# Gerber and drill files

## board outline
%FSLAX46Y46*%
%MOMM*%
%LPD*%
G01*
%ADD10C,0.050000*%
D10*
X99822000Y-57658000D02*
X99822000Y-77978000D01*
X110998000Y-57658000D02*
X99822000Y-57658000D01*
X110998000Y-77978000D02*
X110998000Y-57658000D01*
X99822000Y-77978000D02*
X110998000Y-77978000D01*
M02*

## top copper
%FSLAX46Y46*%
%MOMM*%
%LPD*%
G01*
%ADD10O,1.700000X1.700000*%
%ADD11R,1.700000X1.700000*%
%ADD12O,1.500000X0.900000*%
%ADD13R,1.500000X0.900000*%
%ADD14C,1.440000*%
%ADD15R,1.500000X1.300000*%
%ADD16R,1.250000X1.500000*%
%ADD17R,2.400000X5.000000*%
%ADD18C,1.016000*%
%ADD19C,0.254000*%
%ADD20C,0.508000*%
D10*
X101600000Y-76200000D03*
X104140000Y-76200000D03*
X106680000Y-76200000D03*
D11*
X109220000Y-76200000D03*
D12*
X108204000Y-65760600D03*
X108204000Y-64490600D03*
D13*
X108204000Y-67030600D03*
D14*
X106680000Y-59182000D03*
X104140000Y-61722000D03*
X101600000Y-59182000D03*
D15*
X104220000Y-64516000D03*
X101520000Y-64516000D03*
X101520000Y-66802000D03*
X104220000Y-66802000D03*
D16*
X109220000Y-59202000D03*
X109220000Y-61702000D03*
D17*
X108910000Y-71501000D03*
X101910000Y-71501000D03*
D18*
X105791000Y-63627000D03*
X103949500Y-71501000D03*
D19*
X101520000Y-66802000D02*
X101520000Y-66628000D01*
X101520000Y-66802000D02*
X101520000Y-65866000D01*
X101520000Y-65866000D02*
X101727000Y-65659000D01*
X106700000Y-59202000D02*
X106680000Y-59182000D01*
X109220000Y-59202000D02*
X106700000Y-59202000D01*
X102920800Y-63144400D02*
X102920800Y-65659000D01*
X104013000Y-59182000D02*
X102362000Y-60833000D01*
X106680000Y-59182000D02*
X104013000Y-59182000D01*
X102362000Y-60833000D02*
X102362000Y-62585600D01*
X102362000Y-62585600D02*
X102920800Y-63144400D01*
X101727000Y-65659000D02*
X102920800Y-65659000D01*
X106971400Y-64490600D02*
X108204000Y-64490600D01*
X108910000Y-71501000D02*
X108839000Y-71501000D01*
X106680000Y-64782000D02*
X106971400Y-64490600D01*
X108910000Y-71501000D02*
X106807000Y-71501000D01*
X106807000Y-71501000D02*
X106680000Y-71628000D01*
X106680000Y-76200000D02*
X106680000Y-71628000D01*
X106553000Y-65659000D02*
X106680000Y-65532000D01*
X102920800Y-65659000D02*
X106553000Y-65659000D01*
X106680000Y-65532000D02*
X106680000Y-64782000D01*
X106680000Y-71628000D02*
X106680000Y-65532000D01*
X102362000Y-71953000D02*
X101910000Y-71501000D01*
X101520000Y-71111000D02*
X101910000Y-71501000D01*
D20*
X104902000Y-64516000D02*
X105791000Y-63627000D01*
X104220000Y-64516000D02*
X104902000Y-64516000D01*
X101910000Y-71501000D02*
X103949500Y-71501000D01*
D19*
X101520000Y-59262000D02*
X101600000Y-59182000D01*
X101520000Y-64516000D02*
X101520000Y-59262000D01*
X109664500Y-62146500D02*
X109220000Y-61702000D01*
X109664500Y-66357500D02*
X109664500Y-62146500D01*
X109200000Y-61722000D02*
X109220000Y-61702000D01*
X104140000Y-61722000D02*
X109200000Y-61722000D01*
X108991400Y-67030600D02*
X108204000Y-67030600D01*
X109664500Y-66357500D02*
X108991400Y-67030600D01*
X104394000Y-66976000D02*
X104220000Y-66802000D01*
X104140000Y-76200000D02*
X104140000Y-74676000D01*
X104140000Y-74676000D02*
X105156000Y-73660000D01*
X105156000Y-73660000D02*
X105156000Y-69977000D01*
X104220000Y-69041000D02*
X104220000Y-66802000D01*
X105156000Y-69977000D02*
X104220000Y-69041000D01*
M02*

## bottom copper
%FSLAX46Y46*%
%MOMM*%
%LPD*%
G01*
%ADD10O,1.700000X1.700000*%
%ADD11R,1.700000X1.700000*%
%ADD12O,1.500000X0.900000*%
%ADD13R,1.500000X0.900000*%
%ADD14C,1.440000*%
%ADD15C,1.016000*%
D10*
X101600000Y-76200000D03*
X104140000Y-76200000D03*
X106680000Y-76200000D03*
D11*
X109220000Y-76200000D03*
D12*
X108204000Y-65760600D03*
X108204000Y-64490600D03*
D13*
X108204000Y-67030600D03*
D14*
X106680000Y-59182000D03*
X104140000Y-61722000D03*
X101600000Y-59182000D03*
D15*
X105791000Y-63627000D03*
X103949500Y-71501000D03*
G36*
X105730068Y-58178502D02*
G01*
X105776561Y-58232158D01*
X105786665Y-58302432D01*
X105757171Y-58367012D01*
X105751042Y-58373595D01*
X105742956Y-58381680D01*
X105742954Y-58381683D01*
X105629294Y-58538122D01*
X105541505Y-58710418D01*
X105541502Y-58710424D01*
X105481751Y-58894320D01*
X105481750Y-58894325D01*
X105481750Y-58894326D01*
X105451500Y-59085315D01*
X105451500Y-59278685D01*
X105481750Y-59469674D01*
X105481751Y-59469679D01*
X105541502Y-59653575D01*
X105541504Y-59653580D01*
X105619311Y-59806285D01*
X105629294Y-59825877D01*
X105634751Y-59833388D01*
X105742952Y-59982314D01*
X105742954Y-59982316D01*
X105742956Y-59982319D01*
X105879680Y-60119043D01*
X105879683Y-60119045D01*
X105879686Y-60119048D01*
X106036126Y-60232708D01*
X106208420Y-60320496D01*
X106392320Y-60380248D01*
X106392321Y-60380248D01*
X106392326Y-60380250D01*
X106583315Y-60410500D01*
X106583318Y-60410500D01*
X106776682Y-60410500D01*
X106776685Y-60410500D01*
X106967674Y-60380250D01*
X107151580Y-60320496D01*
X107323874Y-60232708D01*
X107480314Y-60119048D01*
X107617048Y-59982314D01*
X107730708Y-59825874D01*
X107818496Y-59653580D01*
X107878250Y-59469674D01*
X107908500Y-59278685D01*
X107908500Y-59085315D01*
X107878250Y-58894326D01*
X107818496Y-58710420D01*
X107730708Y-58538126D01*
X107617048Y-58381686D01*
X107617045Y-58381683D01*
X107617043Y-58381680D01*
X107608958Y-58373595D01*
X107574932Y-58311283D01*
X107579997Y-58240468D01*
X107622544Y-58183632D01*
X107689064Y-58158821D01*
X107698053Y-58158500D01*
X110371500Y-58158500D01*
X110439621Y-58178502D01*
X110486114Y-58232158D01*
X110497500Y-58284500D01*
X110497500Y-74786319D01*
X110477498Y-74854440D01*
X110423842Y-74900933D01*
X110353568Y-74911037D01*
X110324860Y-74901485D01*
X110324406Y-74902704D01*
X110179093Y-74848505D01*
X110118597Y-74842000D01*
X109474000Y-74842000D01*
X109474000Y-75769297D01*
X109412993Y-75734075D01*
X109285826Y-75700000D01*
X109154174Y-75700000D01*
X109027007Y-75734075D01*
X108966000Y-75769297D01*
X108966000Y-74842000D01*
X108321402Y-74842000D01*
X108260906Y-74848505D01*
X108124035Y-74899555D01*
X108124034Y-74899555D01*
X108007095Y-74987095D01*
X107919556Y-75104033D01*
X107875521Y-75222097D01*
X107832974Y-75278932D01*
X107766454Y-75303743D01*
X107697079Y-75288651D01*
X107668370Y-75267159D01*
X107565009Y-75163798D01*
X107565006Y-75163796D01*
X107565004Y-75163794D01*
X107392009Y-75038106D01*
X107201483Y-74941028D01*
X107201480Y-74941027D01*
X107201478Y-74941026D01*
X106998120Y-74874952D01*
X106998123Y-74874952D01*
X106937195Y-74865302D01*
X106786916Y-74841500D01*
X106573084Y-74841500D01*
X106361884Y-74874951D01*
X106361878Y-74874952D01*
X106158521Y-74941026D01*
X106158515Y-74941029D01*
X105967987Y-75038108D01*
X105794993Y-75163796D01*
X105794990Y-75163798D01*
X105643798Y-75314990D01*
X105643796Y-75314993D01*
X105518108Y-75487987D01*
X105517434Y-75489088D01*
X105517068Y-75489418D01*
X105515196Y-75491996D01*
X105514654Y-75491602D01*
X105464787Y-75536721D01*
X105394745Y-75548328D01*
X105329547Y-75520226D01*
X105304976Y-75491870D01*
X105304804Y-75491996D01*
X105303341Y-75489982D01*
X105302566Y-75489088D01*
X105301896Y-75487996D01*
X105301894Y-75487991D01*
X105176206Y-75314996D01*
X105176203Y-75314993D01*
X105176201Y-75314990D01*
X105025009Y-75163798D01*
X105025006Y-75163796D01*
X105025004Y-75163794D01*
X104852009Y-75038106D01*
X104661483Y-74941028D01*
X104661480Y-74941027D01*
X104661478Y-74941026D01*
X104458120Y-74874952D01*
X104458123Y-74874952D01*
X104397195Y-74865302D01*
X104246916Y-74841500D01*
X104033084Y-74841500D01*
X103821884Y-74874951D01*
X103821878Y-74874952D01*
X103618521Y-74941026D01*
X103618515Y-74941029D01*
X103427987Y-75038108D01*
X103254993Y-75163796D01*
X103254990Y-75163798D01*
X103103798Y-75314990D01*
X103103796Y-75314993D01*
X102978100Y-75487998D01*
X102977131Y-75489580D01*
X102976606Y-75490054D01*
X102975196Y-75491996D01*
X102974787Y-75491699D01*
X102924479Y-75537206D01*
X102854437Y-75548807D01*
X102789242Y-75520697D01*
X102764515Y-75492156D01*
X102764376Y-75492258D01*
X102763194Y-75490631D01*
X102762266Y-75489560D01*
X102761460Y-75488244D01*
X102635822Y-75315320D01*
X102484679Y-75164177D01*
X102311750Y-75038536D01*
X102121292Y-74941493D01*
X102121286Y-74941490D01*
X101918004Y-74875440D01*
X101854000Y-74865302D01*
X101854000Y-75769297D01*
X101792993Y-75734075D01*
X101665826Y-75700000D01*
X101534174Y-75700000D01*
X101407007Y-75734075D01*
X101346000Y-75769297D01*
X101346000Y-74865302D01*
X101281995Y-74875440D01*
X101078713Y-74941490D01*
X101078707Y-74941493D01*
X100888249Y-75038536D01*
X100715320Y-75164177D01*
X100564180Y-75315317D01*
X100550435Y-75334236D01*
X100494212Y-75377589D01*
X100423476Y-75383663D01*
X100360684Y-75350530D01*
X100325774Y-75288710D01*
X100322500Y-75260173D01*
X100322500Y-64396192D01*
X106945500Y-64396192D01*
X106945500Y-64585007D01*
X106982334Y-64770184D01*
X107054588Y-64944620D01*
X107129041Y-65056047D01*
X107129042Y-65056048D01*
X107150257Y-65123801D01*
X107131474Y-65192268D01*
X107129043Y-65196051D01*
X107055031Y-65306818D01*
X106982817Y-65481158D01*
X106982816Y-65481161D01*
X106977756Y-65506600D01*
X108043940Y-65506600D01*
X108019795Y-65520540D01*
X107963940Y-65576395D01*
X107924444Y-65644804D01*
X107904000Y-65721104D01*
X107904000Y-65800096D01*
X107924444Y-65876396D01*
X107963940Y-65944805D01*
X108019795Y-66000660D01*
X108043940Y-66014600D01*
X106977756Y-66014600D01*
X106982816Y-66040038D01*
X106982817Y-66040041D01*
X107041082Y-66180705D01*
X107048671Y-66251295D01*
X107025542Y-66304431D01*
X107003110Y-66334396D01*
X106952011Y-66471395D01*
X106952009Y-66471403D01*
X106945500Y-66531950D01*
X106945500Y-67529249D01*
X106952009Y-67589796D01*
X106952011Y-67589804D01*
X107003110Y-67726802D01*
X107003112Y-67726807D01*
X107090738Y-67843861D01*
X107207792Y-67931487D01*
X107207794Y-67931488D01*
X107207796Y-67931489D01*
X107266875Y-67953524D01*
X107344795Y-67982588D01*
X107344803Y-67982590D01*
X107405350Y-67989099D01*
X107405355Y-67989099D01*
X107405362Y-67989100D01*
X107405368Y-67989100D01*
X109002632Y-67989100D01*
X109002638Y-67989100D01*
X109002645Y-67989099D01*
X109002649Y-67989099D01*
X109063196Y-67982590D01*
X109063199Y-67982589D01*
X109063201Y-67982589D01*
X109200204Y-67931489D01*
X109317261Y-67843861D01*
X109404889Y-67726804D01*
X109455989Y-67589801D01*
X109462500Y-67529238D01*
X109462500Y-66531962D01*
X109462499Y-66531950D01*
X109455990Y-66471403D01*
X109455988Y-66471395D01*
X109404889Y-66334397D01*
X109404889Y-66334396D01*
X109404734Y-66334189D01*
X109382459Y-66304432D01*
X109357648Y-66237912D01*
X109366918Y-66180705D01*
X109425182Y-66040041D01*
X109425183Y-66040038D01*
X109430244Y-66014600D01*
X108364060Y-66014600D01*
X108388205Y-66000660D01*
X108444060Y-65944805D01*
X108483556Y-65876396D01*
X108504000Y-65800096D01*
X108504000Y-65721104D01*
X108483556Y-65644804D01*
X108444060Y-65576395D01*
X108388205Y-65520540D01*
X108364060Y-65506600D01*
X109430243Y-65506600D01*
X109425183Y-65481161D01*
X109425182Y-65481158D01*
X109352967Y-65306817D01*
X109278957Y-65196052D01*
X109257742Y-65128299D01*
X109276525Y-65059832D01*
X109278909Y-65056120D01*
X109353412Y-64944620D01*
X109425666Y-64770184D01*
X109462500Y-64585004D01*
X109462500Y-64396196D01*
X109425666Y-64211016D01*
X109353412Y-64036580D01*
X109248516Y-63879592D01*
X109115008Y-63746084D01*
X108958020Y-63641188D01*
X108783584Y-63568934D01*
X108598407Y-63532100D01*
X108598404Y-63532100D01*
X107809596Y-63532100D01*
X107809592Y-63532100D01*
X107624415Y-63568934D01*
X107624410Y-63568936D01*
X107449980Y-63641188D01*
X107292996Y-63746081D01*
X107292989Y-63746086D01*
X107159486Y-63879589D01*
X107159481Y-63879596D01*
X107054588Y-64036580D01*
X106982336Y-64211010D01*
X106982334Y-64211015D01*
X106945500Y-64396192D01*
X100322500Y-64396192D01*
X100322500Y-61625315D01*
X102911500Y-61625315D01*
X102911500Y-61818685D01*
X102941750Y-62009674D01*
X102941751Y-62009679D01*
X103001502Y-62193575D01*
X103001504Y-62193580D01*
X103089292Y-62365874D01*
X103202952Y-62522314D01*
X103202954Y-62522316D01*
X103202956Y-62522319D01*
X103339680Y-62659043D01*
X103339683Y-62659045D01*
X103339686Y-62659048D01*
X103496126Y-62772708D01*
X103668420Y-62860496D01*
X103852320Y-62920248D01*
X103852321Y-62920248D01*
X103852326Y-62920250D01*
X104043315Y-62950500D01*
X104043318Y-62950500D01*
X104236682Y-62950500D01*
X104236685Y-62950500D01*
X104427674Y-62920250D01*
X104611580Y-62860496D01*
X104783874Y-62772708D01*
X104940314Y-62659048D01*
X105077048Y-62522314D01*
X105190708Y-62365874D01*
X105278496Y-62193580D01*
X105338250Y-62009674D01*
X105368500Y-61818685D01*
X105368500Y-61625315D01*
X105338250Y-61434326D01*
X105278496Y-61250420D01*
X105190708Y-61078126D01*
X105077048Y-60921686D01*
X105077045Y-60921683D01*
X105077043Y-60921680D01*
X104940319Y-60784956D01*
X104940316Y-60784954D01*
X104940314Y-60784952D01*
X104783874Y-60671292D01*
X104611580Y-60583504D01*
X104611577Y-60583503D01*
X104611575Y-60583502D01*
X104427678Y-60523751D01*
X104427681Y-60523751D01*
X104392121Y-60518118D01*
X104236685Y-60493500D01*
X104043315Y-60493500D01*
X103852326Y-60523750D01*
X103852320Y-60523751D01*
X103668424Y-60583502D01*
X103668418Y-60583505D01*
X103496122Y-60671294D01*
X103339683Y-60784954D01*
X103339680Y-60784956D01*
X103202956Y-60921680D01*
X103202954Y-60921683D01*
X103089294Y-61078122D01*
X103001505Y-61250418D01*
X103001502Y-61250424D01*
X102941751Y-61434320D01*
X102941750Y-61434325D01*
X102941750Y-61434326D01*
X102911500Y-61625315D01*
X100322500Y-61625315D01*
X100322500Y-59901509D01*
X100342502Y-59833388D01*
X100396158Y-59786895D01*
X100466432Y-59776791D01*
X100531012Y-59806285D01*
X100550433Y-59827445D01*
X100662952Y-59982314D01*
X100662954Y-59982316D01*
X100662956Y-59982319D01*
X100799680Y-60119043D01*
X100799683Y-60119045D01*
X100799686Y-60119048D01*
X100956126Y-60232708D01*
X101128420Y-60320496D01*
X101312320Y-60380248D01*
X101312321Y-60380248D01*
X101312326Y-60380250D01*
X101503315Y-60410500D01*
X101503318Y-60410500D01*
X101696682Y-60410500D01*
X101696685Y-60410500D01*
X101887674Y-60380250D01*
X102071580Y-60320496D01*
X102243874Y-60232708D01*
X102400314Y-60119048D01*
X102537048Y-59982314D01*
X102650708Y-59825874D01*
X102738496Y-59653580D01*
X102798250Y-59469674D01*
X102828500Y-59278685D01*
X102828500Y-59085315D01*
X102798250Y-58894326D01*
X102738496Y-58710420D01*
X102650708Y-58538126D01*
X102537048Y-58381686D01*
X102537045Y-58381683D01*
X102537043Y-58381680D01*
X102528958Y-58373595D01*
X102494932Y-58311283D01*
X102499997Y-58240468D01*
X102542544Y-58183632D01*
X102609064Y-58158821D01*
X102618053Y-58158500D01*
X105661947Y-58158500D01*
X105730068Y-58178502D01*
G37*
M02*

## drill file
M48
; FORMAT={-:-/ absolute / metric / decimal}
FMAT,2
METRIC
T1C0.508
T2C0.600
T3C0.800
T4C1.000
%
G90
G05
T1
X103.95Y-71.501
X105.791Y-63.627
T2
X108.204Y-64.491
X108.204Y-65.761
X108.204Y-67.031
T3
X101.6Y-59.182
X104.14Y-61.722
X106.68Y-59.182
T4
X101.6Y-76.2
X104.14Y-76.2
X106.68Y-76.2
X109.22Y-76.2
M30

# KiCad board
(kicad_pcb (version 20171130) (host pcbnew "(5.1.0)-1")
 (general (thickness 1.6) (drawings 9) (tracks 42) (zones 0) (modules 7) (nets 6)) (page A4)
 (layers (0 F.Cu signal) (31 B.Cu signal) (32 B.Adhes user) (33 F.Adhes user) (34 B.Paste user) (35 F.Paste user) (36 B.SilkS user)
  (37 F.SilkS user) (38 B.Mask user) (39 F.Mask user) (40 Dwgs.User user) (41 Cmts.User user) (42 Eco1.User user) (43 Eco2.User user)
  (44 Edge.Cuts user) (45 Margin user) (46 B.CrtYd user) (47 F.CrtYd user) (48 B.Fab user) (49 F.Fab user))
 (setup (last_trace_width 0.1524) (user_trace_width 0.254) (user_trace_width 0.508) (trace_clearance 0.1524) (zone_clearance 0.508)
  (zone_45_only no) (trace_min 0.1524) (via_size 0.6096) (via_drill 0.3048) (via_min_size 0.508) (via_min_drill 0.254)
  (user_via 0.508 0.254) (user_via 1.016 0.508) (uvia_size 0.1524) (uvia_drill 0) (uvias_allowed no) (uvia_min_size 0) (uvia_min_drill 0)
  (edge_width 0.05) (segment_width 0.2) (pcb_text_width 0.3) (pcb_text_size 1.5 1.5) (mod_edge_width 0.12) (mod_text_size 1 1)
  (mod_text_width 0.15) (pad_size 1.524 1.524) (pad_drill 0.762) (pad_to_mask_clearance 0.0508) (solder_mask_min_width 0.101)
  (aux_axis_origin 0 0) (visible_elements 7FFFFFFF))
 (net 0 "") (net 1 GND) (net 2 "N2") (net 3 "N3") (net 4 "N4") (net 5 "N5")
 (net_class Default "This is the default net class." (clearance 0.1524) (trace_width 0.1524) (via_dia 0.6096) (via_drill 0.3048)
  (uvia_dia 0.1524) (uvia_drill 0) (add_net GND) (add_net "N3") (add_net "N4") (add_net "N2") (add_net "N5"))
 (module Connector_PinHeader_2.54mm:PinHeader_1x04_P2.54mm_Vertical (layer B.Cu) (at 109.22 76.2 90)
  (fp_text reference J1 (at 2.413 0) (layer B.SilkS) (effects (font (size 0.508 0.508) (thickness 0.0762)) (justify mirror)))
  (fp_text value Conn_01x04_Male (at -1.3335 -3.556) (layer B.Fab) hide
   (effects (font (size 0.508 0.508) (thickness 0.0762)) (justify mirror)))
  (pad 4 thru_hole oval (at 0 -7.62 90) (size 1.7 1.7) (drill 1) (layers *.Cu *.Mask) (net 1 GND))
  (pad 3 thru_hole oval (at 0 -5.08 90) (size 1.7 1.7) (drill 1) (layers *.Cu *.Mask) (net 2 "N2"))
  (pad 2 thru_hole oval (at 0 -2.54 90) (size 1.7 1.7) (drill 1) (layers *.Cu *.Mask) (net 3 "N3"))
  (pad 1 thru_hole rect (at 0 0 90) (size 1.7 1.7) (drill 1) (layers *.Cu *.Mask) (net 1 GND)))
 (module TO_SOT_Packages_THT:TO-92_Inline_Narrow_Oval (layer F.Cu) (at 108.204 67.0306 90)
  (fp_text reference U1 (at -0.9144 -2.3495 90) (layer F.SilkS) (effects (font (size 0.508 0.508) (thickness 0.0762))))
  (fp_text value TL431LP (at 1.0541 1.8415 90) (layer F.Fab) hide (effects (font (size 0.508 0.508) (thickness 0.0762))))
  (pad 2 thru_hole oval (at 1.27 0 270) (size 0.9 1.5) (drill 0.6) (layers *.Cu *.Mask) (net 1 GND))
  (pad 3 thru_hole oval (at 2.54 0 270) (size 0.9 1.5) (drill 0.6) (layers *.Cu *.Mask) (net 3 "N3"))
  (pad 1 thru_hole rect (at 0 0 270) (size 0.9 1.5) (drill 0.6) (layers *.Cu *.Mask) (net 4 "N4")))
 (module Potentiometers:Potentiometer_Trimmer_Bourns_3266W (layer F.Cu) (at 106.68 59.182)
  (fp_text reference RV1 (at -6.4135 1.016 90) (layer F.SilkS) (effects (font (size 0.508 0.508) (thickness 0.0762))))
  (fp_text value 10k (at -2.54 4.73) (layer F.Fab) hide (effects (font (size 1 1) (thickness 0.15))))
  (pad 1 thru_hole circle (at 0 0) (size 1.44 1.44) (drill 0.8) (layers *.Cu *.Mask) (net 3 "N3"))
  (pad 2 thru_hole circle (at -2.54 2.54) (size 1.44 1.44) (drill 0.8) (layers *.Cu *.Mask) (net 4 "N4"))
  (pad 3 thru_hole circle (at -5.08 0) (size 1.44 1.44) (drill 0.8) (layers *.Cu *.Mask) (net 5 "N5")))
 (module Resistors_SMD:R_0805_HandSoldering (layer F.Cu) (at 102.87 64.516 180)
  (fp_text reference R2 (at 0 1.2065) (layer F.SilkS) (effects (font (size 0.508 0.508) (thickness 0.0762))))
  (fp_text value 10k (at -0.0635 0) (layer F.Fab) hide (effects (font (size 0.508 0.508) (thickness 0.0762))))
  (pad 1 smd rect (at -1.35 0 180) (size 1.5 1.3) (layers F.Cu F.Paste F.Mask) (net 1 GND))
  (pad 2 smd rect (at 1.35 0 180) (size 1.5 1.3) (layers F.Cu F.Paste F.Mask) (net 5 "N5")))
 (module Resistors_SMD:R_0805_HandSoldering (layer F.Cu) (at 102.87 66.802)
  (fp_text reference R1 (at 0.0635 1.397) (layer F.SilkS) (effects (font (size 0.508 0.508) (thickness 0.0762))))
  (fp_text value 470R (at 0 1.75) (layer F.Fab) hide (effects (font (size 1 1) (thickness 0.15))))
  (pad 1 smd rect (at -1.35 0) (size 1.5 1.3) (layers F.Cu F.Paste F.Mask) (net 3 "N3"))
  (pad 2 smd rect (at 1.35 0) (size 1.5 1.3) (layers F.Cu F.Paste F.Mask) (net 2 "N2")))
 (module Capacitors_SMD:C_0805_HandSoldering (layer F.Cu) (at 109.22 60.452 270)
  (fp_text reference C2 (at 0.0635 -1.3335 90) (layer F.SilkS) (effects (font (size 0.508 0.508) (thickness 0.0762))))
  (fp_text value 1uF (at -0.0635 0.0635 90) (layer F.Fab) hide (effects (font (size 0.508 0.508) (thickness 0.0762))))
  (pad 1 smd rect (at -1.25 0 270) (size 1.5 1.25) (layers F.Cu F.Paste F.Mask) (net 3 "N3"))
  (pad 2 smd rect (at 1.25 0 270) (size 1.5 1.25) (layers F.Cu F.Paste F.Mask) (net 4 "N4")))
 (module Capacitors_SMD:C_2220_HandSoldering (layer F.Cu) (at 105.41 71.501 180)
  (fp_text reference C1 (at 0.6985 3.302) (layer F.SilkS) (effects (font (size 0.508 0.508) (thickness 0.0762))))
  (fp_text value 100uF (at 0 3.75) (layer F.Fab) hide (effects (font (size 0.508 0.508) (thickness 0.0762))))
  (pad 1 smd rect (at -3.5 0 180) (size 2.4 5) (layers F.Cu F.Paste F.Mask) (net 3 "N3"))
  (pad 2 smd rect (at 3.5 0 180) (size 2.4 5) (layers F.Cu F.Paste F.Mask) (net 1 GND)))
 (gr_line (start 99.822 57.658) (end 99.822 77.978) (layer Edge.Cuts) (width 0.05))
 (gr_line (start 110.998 57.658) (end 99.822 57.658) (layer Edge.Cuts) (width 0.05))
 (gr_line (start 110.998 77.978) (end 110.998 57.658) (layer Edge.Cuts) (width 0.05))
 (gr_line (start 99.822 77.978) (end 110.998 77.978) (layer Edge.Cuts) (width 0.05))
 (segment (start 101.52 66.802) (end 101.52 66.628) (width 0.254) (layer F.Cu) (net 3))
 (segment (start 101.52 66.802) (end 101.52 65.866) (width 0.254) (layer F.Cu) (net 3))
 (segment (start 101.52 65.866) (end 101.727 65.659) (width 0.254) (layer F.Cu) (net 3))
 (segment (start 106.7 59.202) (end 106.68 59.182) (width 0.254) (layer F.Cu) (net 3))
 (segment (start 109.22 59.202) (end 106.7 59.202) (width 0.254) (layer F.Cu) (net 3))
 (segment (start 102.9208 63.1444) (end 102.9208 65.659) (width 0.254) (layer F.Cu) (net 3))
 (segment (start 104.013 59.182) (end 102.362 60.833) (width 0.254) (layer F.Cu) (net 3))
 (segment (start 106.68 59.182) (end 104.013 59.182) (width 0.254) (layer F.Cu) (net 3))
 (segment (start 102.362 60.833) (end 102.362 62.5856) (width 0.254) (layer F.Cu) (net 3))
 (segment (start 102.362 62.5856) (end 102.9208 63.1444) (width 0.254) (layer F.Cu) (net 3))
 (segment (start 101.727 65.659) (end 102.9208 65.659) (width 0.254) (layer F.Cu) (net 3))
 (segment (start 106.9714 64.4906) (end 108.204 64.4906) (width 0.254) (layer F.Cu) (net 3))
 (segment (start 108.91 71.501) (end 108.839 71.501) (width 0.254) (layer F.Cu) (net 3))
 (segment (start 106.68 64.782) (end 106.9714 64.4906) (width 0.254) (layer F.Cu) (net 3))
 (segment (start 108.91 71.501) (end 106.807 71.501) (width 0.254) (layer F.Cu) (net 3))
 (segment (start 106.807 71.501) (end 106.68 71.628) (width 0.254) (layer F.Cu) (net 3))
 (segment (start 106.68 76.2) (end 106.68 71.628) (width 0.254) (layer F.Cu) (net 3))
 (segment (start 106.553 65.659) (end 106.68 65.532) (width 0.254) (layer F.Cu) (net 3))
 (segment (start 102.9208 65.659) (end 106.553 65.659) (width 0.254) (layer F.Cu) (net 3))
 (segment (start 106.68 65.532) (end 106.68 64.782) (width 0.254) (layer F.Cu) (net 3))
 (segment (start 106.68 71.628) (end 106.68 65.532) (width 0.254) (layer F.Cu) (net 3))
 (segment (start 102.362 71.953) (end 101.91 71.501) (width 0.254) (layer F.Cu) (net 1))
 (segment (start 101.52 71.111) (end 101.91 71.501) (width 0.254) (layer F.Cu) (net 1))
 (segment (start 104.902 64.516) (end 105.791 63.627) (width 0.508) (layer F.Cu) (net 1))
 (via (at 105.791 63.627) (size 1.016) (drill 0.508) (layers F.Cu B.Cu) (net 1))
 (segment (start 104.22 64.516) (end 104.902 64.516) (width 0.508) (layer F.Cu) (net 1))
 (via (at 103.9495 71.501) (size 1.016) (drill 0.508) (layers F.Cu B.Cu) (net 1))
 (segment (start 101.91 71.501) (end 103.9495 71.501) (width 0.508) (layer F.Cu) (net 1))
 (segment (start 101.52 59.262) (end 101.6 59.182) (width 0.254) (layer F.Cu) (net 5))
 (segment (start 101.52 64.516) (end 101.52 59.262) (width 0.254) (layer F.Cu) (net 5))
 (segment (start 109.6645 62.1465) (end 109.22 61.702) (width 0.254) (layer F.Cu) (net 4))
 (segment (start 109.6645 66.3575) (end 109.6645 62.1465) (width 0.254) (layer F.Cu) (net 4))
 (segment (start 109.2 61.722) (end 109.22 61.702) (width 0.254) (layer F.Cu) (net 4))
 (segment (start 104.14 61.722) (end 109.2 61.722) (width 0.254) (layer F.Cu) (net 4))
 (segment (start 108.9914 67.0306) (end 108.204 67.0306) (width 0.254) (layer F.Cu) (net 4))
 (segment (start 109.6645 66.3575) (end 108.9914 67.0306) (width 0.254) (layer F.Cu) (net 4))
 (segment (start 104.394 66.976) (end 104.22 66.802) (width 0.254) (layer F.Cu) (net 2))
 (segment (start 104.14 76.2) (end 104.14 74.676) (width 0.254) (layer F.Cu) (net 2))
 (segment (start 104.14 74.676) (end 105.156 73.66) (width 0.254) (layer F.Cu) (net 2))
 (segment (start 105.156 73.66) (end 105.156 69.977) (width 0.254) (layer F.Cu) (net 2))
 (segment (start 104.22 69.041) (end 104.22 66.802) (width 0.254) (layer F.Cu) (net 2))
 (segment (start 105.156 69.977) (end 104.22 69.041) (width 0.254) (layer F.Cu) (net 2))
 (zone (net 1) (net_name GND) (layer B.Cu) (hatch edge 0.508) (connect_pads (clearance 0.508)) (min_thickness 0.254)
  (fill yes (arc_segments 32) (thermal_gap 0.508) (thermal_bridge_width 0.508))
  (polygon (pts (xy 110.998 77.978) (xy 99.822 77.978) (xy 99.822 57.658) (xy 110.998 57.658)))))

